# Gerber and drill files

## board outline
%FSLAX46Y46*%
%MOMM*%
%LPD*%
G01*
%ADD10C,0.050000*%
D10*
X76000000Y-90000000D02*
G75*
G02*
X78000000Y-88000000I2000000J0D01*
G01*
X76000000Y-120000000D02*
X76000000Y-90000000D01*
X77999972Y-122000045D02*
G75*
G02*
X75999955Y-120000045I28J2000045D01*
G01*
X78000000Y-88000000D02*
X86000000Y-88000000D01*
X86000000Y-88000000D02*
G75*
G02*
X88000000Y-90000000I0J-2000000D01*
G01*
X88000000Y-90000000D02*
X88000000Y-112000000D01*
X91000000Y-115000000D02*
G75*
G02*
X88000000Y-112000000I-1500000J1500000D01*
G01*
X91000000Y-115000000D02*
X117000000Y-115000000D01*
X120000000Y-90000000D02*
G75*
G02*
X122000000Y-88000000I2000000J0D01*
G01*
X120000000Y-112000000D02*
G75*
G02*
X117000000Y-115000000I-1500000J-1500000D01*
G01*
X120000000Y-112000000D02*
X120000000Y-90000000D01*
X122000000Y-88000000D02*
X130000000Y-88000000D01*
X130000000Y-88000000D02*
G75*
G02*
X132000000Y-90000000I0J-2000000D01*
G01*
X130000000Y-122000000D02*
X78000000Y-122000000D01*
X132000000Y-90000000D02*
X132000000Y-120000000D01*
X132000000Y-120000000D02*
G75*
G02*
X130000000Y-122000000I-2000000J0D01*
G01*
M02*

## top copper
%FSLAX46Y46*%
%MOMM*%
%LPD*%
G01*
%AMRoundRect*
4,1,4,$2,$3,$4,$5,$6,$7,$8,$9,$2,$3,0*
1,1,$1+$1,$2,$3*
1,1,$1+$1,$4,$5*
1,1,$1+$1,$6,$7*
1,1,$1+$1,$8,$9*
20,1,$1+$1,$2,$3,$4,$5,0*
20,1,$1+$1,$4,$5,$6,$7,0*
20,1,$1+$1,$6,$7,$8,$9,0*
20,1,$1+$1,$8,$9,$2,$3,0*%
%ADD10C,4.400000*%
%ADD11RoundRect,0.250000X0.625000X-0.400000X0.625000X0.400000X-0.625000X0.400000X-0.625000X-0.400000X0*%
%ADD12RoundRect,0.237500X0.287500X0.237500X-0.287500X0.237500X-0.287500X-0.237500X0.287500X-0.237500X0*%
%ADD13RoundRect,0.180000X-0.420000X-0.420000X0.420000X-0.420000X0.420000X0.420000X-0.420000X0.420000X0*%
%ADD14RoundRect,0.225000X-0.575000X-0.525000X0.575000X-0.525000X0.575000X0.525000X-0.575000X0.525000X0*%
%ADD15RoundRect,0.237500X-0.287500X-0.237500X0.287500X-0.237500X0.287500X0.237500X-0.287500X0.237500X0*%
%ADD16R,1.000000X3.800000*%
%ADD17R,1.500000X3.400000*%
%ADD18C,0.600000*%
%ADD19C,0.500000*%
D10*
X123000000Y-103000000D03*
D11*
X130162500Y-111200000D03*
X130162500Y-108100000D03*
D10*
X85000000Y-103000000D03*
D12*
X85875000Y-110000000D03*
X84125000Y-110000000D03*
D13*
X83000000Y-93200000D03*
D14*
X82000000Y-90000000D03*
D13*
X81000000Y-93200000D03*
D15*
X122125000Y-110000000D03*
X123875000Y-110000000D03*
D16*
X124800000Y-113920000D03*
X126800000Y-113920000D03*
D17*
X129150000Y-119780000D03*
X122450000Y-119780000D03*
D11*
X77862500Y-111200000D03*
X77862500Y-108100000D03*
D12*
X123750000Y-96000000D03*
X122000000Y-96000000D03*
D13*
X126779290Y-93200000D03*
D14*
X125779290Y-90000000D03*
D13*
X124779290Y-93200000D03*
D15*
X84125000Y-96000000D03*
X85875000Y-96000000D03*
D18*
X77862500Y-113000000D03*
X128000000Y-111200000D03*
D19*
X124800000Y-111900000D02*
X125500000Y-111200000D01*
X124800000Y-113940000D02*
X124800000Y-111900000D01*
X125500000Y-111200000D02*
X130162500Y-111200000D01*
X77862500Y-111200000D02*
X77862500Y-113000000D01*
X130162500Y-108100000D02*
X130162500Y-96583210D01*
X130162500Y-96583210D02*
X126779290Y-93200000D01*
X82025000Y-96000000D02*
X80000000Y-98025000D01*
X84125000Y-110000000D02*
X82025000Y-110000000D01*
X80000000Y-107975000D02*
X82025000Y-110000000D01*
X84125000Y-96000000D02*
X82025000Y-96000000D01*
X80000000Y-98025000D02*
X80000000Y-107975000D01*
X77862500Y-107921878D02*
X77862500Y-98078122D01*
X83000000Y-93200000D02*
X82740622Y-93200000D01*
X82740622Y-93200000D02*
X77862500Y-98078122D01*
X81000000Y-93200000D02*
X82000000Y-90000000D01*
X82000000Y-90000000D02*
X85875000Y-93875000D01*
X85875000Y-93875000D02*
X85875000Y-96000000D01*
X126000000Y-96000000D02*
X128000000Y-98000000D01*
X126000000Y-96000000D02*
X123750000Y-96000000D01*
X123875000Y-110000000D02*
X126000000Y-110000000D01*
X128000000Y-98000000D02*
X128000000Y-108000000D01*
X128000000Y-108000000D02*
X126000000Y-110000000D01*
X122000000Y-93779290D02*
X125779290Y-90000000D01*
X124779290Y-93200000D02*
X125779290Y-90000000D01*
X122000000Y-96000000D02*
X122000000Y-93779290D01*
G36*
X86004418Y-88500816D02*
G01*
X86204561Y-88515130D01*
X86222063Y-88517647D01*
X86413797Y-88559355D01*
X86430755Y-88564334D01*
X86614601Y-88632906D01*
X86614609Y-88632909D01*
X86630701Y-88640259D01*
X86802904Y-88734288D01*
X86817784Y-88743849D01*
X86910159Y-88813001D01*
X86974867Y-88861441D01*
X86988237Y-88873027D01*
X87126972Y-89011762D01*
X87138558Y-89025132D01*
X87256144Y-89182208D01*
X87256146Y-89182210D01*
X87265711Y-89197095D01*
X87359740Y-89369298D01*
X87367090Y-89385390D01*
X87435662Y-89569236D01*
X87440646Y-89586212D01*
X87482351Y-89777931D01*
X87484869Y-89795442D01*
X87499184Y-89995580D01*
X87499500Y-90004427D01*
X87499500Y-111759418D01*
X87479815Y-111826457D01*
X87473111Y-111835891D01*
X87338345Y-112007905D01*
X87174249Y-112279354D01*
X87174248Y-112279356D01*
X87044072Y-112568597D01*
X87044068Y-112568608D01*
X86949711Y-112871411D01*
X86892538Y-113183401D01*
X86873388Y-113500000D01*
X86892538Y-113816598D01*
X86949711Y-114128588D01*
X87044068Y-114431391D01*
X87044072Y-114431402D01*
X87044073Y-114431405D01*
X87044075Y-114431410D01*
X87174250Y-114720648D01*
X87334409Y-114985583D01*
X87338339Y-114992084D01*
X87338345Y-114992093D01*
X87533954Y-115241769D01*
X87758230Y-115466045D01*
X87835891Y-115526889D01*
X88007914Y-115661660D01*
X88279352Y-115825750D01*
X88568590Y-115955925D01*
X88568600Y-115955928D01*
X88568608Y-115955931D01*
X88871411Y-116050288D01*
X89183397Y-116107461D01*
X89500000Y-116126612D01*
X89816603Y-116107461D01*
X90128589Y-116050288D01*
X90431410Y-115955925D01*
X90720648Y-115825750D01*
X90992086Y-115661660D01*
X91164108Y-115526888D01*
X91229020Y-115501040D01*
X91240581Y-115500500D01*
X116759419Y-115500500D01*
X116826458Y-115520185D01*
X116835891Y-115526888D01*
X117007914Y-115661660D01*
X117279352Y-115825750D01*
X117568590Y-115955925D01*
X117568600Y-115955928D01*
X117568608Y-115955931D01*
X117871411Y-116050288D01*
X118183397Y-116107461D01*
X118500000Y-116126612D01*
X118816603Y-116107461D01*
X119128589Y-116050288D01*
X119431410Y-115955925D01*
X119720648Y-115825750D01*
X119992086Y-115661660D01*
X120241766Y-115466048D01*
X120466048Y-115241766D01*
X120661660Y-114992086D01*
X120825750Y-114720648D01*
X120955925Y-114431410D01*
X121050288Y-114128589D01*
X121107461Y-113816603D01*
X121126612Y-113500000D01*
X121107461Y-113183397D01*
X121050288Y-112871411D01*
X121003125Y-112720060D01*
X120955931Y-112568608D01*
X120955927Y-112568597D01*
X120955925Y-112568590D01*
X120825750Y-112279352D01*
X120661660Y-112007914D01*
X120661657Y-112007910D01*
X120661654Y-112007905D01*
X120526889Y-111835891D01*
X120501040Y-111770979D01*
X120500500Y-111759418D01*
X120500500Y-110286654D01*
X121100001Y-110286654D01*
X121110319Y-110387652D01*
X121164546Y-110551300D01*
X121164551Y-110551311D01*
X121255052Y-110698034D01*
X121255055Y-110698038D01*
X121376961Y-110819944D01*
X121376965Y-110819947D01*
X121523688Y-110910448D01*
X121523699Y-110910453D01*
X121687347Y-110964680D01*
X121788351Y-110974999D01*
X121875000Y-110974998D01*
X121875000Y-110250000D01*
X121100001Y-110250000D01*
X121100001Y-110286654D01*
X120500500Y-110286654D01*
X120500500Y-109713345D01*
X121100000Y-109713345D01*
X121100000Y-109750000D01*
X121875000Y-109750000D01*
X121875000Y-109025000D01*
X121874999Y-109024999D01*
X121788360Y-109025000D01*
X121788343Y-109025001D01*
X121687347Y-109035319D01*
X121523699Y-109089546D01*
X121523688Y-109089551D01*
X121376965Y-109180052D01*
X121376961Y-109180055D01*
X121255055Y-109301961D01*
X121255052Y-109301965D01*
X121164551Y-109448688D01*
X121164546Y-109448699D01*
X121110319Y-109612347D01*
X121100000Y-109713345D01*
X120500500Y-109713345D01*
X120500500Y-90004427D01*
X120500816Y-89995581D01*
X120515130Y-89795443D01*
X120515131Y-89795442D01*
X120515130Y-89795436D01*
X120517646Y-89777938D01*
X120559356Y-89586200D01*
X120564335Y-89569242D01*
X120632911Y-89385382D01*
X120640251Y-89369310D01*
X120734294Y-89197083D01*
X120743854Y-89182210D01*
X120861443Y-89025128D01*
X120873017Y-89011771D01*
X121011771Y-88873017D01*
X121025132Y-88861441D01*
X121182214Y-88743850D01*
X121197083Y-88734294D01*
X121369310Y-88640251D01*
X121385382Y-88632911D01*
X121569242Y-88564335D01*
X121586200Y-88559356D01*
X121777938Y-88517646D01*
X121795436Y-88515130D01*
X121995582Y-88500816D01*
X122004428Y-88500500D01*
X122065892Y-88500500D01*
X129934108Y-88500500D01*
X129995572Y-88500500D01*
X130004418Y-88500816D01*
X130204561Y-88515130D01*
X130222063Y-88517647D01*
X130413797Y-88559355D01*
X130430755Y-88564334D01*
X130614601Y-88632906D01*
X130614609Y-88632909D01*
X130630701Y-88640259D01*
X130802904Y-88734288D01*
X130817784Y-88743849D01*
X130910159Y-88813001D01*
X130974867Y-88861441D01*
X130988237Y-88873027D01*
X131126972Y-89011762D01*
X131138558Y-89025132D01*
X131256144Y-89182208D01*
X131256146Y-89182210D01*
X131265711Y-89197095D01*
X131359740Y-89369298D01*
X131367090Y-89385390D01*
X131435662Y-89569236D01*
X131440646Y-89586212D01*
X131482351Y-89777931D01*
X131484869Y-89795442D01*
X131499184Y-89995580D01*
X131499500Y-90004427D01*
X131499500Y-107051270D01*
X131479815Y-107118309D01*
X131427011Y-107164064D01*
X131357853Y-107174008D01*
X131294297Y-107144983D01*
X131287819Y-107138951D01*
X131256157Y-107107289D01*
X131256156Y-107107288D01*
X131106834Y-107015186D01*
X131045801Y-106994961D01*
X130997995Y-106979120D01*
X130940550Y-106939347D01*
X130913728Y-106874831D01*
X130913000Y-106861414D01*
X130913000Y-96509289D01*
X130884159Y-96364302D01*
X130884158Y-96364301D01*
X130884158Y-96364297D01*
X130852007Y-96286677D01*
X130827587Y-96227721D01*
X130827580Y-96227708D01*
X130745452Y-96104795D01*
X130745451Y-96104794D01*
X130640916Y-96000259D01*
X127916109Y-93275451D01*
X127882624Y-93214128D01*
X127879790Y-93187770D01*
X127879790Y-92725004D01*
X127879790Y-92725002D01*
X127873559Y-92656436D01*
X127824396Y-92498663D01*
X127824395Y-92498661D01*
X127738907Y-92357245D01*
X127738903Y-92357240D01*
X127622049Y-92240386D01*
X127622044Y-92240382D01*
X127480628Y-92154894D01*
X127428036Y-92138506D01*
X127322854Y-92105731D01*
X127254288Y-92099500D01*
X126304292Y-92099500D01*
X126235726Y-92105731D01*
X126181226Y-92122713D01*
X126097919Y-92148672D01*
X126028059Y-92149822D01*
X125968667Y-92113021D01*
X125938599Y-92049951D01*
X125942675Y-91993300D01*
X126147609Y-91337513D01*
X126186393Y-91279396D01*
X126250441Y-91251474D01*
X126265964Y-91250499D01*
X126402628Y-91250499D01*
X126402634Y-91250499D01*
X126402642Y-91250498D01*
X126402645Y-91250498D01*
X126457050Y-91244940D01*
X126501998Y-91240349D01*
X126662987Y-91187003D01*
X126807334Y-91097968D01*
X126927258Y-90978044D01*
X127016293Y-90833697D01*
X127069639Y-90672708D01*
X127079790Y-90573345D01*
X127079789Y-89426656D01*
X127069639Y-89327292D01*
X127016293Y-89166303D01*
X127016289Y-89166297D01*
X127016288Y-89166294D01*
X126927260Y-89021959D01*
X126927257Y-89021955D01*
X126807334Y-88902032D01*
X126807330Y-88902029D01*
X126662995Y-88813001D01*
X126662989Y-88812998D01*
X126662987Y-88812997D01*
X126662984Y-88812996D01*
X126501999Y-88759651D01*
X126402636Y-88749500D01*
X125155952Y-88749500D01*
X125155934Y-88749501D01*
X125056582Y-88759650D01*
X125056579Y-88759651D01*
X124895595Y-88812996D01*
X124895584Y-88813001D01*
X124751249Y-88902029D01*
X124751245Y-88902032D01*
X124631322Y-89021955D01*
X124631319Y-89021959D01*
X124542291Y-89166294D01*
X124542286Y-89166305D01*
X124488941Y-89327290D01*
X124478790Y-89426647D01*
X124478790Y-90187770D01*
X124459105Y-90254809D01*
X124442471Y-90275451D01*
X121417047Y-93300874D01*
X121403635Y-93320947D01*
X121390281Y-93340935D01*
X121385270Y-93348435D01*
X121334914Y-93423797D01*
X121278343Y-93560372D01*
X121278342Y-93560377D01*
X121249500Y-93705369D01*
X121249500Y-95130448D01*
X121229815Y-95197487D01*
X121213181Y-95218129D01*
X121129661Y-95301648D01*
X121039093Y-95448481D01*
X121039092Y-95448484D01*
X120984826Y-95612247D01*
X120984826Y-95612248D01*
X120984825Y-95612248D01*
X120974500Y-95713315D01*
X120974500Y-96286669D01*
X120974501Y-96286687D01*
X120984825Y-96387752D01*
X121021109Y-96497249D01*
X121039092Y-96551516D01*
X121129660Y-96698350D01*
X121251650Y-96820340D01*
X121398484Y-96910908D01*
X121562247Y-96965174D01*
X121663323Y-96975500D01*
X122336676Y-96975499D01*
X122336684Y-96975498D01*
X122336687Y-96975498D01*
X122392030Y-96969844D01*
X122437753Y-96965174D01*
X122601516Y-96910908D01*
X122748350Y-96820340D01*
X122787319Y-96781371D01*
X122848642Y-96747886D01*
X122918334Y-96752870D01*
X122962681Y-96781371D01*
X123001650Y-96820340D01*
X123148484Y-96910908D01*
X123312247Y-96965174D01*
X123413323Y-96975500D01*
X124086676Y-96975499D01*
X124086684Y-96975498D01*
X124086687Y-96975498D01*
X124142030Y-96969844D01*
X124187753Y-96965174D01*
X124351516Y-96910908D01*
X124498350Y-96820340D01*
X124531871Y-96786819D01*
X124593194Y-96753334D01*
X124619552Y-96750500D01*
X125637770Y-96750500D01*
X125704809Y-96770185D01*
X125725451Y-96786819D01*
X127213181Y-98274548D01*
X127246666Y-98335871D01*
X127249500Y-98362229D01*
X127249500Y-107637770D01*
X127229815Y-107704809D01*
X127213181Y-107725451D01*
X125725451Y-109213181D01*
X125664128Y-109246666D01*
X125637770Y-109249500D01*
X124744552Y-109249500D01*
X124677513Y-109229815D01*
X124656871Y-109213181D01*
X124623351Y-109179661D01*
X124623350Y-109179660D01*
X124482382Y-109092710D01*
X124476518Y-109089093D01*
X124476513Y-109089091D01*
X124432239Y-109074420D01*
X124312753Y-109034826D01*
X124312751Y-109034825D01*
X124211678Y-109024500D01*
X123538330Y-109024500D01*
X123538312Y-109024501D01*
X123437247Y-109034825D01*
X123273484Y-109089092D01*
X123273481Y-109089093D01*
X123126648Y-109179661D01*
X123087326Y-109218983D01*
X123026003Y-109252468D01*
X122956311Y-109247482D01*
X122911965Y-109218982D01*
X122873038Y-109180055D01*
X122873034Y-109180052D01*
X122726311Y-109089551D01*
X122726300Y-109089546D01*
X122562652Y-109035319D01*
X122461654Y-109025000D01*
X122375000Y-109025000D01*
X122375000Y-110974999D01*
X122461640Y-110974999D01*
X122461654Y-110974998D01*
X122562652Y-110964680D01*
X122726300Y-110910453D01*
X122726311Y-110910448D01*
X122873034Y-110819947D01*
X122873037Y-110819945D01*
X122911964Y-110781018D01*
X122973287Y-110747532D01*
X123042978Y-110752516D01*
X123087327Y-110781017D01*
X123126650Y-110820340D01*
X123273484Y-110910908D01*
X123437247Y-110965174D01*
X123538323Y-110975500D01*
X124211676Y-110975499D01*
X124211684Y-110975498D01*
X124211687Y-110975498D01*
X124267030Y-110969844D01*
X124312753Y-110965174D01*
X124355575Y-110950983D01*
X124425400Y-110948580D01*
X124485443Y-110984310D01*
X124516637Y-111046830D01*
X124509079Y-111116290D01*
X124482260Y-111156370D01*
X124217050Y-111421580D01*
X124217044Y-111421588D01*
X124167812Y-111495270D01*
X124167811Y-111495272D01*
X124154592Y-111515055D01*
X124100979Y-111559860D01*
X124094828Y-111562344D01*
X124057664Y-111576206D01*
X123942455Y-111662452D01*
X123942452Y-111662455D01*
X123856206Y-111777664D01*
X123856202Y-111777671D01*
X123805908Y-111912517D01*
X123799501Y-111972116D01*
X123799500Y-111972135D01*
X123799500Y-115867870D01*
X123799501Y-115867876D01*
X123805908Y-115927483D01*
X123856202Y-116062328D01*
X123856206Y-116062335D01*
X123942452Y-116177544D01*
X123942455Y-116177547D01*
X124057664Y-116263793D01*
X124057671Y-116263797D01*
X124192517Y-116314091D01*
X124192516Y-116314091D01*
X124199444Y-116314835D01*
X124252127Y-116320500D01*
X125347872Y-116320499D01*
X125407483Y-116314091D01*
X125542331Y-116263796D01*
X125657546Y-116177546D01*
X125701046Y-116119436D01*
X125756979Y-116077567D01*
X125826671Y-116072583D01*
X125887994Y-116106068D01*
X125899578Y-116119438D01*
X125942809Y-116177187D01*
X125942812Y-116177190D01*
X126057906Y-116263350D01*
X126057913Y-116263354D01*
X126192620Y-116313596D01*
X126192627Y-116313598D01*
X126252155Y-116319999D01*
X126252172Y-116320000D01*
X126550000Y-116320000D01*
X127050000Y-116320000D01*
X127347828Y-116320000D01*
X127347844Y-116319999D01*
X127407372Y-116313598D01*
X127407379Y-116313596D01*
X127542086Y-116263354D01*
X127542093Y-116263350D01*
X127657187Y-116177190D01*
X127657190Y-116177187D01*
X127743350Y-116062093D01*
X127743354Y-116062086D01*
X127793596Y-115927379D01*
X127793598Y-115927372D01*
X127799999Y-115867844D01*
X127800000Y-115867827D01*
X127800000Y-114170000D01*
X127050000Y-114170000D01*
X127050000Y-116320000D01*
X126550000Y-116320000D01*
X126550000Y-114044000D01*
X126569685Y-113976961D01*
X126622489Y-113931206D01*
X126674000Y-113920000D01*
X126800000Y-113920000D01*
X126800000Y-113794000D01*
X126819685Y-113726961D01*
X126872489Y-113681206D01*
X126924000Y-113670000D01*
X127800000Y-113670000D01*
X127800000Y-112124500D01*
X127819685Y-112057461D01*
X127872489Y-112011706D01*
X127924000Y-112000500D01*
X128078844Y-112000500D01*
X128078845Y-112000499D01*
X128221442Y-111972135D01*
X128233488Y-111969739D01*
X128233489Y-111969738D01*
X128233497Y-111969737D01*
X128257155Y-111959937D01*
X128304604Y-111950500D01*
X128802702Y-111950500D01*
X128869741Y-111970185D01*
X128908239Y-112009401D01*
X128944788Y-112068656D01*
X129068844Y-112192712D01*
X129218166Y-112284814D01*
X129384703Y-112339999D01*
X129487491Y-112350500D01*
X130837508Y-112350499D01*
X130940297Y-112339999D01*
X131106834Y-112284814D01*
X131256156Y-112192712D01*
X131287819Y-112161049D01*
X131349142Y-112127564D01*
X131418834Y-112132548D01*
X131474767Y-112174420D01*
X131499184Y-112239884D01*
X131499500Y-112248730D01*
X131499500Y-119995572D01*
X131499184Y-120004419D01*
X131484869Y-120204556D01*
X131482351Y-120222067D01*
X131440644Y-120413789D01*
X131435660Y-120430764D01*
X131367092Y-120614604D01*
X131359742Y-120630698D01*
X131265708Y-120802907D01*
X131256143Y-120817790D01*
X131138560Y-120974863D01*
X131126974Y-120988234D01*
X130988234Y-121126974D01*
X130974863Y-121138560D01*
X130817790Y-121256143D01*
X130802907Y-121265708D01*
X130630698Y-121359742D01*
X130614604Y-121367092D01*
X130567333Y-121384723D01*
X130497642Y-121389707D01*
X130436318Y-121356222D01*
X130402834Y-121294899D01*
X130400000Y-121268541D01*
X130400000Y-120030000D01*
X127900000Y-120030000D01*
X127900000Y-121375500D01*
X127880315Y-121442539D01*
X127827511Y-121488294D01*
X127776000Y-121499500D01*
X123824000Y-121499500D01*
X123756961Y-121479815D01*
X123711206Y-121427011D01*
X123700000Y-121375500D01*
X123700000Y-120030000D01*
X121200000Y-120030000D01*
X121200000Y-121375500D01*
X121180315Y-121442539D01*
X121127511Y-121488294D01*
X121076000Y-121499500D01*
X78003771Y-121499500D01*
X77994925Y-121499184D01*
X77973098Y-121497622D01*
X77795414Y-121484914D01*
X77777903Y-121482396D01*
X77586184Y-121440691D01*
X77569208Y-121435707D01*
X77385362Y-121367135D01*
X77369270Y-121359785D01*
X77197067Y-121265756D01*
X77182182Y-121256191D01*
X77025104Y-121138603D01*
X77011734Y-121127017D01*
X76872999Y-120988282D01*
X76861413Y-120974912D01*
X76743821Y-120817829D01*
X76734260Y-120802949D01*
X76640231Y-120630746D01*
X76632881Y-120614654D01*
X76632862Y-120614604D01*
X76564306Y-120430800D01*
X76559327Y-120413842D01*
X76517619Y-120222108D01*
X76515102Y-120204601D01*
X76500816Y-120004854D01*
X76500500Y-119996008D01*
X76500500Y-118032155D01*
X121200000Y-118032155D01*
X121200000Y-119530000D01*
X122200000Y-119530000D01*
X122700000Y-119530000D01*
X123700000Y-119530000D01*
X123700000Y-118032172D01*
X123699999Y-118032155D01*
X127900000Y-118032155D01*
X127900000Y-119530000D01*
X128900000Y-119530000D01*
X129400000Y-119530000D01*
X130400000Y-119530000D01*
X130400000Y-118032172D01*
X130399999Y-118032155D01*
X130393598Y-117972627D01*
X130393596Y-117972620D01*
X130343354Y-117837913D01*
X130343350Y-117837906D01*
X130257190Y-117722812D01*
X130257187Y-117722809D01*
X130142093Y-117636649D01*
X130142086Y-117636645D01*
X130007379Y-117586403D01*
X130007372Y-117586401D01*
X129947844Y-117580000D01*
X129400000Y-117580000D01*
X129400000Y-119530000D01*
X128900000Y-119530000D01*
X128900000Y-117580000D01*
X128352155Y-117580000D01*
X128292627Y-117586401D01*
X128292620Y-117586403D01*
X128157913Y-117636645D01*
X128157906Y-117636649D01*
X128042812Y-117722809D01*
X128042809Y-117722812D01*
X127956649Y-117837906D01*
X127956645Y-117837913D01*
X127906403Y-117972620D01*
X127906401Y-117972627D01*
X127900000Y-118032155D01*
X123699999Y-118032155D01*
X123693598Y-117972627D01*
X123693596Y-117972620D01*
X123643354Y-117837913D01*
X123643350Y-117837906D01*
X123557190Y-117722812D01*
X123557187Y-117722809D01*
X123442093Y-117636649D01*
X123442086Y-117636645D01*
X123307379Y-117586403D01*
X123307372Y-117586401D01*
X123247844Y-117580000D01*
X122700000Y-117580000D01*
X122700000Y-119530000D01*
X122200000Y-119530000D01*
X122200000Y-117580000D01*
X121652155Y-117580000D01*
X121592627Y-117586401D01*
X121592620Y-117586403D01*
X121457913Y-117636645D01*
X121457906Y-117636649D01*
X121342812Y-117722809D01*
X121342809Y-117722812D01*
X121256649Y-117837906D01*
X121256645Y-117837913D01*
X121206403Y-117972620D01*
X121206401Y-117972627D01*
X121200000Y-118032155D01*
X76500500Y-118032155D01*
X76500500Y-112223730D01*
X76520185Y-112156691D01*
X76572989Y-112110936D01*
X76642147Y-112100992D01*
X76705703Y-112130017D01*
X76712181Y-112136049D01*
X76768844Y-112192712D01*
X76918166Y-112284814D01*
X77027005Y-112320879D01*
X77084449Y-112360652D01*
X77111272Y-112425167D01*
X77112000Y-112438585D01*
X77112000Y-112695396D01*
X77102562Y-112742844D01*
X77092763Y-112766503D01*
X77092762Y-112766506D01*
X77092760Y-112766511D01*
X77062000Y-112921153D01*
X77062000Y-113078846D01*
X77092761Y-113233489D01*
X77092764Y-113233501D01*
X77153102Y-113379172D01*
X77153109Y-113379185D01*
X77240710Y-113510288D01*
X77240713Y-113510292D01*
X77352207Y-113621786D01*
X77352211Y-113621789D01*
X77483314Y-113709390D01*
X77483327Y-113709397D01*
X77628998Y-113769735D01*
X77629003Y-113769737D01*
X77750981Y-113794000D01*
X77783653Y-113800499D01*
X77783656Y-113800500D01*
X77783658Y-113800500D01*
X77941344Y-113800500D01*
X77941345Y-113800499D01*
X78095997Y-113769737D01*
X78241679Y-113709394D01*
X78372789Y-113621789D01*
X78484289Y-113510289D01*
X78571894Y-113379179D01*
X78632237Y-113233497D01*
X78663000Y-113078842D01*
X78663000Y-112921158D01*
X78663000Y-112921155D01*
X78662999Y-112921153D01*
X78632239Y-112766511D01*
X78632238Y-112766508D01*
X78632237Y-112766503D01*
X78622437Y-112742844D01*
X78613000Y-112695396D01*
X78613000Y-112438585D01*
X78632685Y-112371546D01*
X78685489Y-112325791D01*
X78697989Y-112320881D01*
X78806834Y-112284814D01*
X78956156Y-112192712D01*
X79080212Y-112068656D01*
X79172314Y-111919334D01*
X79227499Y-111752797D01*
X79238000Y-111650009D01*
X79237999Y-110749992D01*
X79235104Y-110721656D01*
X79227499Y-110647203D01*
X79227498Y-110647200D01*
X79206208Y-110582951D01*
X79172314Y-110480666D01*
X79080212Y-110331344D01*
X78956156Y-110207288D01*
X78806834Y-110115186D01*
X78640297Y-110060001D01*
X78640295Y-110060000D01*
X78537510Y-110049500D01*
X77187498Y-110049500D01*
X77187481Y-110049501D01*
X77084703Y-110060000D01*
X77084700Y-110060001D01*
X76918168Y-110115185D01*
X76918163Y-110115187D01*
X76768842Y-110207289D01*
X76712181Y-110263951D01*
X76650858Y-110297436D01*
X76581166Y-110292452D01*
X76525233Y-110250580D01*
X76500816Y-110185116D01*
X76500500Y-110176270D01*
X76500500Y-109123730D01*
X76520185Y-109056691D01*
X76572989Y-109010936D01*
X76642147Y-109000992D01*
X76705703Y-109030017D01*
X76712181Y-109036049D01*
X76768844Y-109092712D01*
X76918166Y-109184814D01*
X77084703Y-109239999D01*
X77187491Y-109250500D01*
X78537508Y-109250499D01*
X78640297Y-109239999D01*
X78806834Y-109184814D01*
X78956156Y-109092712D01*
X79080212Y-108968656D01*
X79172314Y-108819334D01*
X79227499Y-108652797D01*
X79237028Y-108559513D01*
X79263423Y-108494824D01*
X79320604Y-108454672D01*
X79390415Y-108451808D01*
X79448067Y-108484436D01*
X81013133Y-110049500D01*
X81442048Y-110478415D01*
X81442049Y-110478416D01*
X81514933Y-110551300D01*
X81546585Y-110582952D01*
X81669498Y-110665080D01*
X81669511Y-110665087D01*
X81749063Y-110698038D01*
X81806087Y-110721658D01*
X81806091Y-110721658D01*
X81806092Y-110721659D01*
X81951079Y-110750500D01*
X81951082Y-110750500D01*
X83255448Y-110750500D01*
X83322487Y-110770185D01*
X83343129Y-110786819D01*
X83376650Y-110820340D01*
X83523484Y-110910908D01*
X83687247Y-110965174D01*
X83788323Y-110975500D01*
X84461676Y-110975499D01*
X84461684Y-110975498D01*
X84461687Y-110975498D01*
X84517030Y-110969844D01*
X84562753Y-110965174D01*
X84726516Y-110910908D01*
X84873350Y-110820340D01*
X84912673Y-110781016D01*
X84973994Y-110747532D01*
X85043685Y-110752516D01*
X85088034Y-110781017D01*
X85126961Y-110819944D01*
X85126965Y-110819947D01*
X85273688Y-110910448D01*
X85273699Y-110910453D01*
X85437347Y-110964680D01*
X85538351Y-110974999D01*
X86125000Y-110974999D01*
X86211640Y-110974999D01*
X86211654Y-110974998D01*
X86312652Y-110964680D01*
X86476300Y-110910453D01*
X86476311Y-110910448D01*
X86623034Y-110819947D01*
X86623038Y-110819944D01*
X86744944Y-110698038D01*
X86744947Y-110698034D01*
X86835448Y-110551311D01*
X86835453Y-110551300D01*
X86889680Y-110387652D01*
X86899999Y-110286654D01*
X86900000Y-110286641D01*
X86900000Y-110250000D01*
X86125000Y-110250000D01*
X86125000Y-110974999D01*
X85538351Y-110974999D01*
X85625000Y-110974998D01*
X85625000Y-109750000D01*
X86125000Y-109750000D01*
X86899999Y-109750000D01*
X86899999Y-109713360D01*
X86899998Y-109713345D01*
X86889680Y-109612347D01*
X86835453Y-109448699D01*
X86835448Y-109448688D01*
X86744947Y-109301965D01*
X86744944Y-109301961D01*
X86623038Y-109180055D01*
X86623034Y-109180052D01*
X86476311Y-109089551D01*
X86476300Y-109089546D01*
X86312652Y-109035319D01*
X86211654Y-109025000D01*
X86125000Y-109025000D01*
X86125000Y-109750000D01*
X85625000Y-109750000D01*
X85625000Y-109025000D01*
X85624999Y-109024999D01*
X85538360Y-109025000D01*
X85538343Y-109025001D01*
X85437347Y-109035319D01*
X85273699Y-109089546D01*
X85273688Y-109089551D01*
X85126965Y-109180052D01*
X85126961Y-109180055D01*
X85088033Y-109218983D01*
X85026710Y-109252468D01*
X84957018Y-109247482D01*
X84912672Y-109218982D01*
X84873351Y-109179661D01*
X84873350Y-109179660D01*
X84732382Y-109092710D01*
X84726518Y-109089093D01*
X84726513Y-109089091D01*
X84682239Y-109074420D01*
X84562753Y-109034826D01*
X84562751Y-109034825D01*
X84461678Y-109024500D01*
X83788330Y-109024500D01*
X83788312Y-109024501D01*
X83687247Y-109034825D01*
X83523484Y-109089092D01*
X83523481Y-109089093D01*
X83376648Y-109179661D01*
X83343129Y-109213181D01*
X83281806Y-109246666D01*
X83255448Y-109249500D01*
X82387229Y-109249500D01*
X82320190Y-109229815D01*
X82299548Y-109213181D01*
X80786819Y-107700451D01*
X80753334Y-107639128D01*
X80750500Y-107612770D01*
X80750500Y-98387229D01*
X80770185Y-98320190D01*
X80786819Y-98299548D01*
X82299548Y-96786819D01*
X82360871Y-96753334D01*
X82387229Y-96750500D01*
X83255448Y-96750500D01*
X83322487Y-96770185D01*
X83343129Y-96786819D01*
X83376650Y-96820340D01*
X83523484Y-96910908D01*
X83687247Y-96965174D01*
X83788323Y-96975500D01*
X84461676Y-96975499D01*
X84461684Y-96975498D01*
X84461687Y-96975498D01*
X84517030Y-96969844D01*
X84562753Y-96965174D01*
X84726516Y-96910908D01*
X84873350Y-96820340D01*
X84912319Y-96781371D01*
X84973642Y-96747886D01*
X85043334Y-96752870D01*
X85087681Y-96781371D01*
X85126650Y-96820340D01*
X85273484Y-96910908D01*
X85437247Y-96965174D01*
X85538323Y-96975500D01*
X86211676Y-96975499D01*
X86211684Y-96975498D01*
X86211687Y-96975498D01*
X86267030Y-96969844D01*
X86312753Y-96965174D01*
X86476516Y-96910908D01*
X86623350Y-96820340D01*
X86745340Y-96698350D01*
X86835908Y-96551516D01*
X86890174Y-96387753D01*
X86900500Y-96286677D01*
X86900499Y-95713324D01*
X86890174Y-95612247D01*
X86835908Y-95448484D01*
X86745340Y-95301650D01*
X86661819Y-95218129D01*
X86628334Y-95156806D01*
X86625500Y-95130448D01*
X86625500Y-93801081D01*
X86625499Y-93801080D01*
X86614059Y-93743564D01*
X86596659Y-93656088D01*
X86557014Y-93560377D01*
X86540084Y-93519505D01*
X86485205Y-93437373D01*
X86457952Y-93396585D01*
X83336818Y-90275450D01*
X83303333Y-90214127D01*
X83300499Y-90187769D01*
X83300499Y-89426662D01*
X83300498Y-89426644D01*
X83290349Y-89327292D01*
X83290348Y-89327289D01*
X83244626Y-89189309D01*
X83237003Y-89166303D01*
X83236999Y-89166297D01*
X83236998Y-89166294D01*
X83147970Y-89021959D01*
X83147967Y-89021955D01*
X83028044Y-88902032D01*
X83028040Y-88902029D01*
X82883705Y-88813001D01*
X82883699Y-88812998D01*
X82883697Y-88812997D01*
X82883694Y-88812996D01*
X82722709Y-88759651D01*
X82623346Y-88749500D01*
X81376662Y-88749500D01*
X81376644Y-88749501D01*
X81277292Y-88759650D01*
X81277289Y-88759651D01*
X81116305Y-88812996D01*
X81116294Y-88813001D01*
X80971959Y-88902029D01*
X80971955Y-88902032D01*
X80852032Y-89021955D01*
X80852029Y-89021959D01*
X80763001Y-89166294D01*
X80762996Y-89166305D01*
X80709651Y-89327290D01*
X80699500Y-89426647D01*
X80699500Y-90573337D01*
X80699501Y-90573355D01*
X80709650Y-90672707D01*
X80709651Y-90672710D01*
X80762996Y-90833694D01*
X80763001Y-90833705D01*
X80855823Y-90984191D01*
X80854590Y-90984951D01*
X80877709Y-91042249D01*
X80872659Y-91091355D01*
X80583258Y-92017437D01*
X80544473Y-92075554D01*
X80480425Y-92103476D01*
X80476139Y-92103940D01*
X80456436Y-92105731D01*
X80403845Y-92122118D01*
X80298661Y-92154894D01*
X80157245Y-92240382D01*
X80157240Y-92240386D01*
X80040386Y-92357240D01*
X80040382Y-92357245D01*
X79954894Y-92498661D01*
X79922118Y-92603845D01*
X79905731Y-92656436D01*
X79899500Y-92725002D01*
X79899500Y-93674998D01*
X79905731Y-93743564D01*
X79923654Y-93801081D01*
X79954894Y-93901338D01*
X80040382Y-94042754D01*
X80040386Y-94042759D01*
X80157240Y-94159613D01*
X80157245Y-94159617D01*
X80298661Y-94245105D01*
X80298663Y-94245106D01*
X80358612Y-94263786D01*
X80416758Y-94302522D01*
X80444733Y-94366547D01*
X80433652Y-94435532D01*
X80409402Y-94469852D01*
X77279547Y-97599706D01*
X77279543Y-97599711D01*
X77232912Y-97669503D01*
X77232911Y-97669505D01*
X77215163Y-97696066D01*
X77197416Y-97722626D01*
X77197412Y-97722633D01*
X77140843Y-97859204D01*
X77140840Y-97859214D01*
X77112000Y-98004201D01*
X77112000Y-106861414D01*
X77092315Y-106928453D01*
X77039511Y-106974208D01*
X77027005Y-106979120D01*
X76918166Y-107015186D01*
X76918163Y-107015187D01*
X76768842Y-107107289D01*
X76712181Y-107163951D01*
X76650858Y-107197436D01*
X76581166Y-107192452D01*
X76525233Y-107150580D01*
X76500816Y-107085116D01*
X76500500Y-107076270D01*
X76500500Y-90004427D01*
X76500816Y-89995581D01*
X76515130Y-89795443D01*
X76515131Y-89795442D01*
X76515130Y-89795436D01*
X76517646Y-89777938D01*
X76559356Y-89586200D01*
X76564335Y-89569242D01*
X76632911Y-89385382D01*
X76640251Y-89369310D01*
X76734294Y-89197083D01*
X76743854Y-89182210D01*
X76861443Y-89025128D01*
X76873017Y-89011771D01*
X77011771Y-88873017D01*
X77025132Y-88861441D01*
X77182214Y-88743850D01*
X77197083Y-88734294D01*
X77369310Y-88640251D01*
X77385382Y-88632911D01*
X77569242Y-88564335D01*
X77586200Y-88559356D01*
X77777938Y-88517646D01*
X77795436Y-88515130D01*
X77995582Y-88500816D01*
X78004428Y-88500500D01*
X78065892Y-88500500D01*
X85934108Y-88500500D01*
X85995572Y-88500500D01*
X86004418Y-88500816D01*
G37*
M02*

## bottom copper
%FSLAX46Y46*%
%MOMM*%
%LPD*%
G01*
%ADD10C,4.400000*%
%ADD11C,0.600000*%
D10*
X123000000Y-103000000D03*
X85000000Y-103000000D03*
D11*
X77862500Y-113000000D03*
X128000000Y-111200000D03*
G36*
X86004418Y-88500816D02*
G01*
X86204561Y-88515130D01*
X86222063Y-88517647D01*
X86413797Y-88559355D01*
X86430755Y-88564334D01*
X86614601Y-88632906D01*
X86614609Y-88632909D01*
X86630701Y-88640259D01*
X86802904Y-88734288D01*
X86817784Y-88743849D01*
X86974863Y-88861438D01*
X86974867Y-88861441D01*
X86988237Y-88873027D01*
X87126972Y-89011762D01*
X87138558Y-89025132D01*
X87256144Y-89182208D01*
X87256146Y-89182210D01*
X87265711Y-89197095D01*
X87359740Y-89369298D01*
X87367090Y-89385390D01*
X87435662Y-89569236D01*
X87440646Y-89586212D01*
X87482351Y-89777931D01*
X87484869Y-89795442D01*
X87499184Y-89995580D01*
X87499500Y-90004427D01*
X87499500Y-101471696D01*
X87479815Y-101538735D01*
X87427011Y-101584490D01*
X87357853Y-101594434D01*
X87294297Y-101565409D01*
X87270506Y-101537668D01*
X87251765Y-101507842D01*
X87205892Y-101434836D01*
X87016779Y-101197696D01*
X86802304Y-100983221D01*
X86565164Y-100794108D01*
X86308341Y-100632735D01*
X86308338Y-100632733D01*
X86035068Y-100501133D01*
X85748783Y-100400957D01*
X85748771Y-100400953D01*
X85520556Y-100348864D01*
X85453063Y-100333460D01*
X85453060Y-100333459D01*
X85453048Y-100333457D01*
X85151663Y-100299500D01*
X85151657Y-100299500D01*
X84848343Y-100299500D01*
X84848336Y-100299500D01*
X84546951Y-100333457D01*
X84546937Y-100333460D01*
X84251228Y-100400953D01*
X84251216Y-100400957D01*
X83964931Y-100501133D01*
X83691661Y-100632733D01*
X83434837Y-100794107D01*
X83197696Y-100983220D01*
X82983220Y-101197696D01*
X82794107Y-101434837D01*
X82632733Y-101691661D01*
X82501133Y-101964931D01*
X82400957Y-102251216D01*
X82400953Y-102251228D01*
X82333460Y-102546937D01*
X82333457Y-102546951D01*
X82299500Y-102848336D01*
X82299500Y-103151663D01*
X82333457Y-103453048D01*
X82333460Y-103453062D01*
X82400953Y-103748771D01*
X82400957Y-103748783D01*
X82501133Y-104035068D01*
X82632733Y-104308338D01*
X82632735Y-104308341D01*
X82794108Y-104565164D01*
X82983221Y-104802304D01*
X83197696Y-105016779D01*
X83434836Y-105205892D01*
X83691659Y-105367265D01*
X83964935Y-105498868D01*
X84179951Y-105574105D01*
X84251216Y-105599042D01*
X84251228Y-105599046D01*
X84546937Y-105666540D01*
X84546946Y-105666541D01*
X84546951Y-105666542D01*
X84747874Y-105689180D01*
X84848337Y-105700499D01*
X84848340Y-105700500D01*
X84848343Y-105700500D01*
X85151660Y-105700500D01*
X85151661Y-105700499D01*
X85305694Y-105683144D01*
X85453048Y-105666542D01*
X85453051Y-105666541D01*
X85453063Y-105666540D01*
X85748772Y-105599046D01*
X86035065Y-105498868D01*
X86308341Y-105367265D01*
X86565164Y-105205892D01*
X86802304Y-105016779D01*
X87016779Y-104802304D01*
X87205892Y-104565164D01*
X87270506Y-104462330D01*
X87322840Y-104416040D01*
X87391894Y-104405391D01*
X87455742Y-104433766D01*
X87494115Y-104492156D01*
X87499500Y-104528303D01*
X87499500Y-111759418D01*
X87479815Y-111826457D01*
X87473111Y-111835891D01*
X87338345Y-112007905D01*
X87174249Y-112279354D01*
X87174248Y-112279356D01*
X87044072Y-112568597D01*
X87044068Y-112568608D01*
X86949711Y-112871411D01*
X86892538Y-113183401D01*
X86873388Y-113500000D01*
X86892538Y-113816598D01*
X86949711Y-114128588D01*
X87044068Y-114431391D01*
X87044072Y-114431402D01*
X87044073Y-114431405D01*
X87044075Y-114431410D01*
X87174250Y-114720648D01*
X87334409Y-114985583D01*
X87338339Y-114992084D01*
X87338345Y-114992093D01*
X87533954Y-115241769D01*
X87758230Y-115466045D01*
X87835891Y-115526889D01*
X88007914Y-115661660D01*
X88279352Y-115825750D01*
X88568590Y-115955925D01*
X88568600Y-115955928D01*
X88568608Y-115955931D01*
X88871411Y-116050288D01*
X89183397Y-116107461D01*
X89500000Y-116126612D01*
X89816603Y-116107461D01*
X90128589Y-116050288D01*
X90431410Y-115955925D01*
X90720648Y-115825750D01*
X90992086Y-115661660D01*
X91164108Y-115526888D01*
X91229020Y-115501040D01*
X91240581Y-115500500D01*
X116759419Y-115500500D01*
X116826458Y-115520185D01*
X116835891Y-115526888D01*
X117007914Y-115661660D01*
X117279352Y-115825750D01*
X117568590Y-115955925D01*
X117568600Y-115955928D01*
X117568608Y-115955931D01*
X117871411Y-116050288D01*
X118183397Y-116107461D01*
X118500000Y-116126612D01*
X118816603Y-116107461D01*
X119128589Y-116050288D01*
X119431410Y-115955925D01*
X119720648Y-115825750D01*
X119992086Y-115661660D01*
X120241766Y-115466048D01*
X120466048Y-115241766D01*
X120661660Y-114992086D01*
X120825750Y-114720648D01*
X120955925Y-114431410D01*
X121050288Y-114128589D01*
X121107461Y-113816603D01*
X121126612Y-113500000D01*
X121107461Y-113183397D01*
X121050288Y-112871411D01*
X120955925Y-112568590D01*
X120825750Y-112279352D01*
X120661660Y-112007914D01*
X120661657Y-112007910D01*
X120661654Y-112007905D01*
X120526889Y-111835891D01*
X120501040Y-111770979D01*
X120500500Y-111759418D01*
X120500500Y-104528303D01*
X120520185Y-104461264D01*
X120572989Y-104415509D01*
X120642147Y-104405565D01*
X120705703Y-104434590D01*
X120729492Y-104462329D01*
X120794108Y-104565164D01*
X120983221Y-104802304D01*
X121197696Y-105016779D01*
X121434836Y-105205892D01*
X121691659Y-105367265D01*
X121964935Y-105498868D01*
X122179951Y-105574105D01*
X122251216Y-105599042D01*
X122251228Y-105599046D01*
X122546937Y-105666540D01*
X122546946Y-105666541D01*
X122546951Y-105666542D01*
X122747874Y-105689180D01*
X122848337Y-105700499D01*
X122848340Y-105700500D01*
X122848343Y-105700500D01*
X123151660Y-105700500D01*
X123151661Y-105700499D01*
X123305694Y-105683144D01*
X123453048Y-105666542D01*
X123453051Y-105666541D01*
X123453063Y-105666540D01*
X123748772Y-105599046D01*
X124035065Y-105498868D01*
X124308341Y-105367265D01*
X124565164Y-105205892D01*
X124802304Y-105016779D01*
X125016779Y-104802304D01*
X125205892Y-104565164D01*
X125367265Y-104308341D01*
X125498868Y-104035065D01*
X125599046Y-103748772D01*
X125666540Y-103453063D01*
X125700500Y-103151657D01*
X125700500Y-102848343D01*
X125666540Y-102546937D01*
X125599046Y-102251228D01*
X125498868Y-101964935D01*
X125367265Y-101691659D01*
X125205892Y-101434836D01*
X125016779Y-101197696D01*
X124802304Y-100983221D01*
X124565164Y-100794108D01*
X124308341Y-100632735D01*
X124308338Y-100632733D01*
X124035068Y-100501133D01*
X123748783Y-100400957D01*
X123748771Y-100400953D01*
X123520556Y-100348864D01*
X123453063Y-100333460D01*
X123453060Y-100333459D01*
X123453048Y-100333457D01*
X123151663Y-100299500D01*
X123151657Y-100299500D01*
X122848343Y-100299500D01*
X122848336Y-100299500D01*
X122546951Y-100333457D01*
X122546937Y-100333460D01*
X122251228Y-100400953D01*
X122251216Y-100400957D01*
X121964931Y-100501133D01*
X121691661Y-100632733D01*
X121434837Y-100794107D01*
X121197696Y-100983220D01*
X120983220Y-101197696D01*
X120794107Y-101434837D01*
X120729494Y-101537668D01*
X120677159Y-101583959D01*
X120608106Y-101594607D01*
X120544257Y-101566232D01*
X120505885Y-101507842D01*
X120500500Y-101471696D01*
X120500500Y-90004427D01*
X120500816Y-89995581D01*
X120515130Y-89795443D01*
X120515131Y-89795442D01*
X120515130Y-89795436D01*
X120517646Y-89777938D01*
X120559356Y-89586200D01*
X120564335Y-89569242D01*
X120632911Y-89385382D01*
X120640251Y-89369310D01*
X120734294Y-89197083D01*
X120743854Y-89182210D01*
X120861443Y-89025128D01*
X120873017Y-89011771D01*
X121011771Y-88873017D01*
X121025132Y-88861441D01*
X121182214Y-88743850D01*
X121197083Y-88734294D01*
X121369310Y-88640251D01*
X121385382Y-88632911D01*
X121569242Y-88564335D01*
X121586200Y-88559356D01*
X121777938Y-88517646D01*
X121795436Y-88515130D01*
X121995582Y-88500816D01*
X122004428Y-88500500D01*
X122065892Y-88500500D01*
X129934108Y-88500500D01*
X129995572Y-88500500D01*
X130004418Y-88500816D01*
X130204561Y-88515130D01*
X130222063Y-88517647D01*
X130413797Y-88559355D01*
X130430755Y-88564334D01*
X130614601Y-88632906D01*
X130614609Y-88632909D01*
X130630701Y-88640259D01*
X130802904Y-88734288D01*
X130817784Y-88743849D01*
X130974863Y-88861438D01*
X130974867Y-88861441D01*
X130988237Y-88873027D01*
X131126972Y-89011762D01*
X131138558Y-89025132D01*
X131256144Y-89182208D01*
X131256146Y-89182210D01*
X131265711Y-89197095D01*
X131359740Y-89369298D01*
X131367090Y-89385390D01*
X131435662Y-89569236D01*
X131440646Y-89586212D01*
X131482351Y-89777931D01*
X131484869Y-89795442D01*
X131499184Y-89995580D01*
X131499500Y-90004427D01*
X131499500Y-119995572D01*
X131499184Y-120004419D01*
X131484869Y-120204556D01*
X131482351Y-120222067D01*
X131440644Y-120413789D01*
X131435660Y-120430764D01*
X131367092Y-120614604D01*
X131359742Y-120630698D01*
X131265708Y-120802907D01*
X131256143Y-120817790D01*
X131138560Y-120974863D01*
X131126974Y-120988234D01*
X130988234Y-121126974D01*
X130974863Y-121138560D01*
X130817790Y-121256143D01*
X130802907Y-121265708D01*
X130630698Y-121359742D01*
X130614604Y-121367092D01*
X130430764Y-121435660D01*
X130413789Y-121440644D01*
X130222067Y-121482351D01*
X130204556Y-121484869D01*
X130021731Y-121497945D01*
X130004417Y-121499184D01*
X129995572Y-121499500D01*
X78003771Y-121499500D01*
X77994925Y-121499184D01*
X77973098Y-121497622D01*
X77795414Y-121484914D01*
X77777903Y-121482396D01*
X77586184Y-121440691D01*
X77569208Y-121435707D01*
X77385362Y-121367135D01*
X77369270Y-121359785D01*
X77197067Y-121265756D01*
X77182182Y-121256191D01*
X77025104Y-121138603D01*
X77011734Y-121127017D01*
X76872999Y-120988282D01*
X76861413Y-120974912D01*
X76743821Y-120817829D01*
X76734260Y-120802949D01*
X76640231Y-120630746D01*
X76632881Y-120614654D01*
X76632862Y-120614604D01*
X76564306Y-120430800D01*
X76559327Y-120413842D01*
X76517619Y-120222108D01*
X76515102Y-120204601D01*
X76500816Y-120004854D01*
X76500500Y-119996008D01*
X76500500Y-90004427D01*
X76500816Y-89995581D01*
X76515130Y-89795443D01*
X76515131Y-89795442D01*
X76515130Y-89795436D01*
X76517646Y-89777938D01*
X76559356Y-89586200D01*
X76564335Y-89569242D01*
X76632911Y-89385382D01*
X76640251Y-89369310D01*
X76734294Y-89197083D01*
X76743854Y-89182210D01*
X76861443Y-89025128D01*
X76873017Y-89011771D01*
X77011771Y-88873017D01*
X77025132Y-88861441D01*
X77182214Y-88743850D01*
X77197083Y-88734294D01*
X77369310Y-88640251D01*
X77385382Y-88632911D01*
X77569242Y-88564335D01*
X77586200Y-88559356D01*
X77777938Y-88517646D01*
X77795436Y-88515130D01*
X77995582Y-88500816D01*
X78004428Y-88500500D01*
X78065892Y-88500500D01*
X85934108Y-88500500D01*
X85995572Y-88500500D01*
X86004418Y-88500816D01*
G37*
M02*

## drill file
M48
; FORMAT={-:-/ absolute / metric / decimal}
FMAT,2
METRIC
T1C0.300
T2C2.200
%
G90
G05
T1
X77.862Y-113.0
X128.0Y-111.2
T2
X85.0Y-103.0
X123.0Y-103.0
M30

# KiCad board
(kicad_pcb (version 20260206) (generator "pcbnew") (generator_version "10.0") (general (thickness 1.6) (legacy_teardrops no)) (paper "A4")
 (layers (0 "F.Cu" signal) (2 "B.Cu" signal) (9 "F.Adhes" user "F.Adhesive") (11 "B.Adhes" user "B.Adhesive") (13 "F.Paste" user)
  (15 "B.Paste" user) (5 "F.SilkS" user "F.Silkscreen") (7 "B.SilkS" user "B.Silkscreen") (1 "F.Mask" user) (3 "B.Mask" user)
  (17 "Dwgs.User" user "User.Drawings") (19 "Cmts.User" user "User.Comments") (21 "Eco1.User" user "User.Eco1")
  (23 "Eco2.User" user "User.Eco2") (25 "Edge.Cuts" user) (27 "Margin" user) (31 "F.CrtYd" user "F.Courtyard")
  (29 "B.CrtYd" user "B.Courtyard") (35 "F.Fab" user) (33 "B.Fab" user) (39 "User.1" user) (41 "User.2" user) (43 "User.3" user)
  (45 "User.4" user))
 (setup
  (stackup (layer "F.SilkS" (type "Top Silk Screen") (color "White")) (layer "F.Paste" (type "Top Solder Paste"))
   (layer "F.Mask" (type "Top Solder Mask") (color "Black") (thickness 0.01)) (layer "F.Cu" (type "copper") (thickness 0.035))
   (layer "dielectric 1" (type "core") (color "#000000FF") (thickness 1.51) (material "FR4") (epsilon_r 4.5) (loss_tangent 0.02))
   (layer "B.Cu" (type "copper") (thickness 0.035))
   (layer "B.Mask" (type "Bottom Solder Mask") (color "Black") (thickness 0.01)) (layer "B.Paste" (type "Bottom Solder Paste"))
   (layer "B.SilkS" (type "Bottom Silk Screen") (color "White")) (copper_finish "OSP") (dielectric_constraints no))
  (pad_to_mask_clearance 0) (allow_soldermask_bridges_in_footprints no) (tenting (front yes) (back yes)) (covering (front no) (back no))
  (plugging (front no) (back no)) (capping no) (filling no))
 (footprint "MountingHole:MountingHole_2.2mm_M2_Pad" (layer "F.Cu") (at 123 103)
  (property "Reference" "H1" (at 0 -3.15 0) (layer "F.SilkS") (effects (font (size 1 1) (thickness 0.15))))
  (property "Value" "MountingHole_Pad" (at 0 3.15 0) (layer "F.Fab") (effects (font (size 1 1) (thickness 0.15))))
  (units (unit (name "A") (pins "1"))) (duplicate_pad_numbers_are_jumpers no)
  (pad "1" thru_hole circle (at 0 0) (size 4.4 4.4) (drill 2.2) (layers "*.Cu" "*.Mask") (remove_unused_layers no) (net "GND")
   (zone_connect 2)))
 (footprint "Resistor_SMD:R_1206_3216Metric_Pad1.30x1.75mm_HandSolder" (layer "F.Cu") (at 130.1625 109.65 90)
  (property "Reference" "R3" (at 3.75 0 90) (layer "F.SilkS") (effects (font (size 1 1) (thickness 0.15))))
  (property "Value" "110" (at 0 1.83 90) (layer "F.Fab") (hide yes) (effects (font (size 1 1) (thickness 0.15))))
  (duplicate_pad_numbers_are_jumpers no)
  (pad "1" smd roundrect (at -1.55 0 90) (size 1.3 1.75) (layers "F.Cu" "F.Mask" "F.Paste") (roundrect_rratio 0.192308) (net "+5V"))
  (pad "2" smd roundrect (at 1.55 0 90) (size 1.3 1.75) (layers "F.Cu" "F.Mask" "F.Paste") (roundrect_rratio 0.192308) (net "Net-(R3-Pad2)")))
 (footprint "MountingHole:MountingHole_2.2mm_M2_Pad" (layer "F.Cu") (at 85 103)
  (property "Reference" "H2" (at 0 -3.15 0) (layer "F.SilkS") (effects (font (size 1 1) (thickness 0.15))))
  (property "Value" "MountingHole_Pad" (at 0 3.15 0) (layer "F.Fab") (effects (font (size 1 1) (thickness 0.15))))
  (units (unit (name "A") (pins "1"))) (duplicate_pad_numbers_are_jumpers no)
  (pad "1" thru_hole circle (at 0 0) (size 4.4 4.4) (drill 2.2) (layers "*.Cu" "*.Mask") (remove_unused_layers no) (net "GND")
   (zone_connect 2)))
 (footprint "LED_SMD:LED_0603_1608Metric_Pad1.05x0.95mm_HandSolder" (layer "F.Cu") (at 85 110 180)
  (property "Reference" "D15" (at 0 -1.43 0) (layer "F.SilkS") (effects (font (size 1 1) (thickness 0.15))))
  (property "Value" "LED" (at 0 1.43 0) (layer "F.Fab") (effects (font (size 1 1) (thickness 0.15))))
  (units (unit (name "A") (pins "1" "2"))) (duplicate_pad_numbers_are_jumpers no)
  (pad "1" smd roundrect (at -0.875 0 180) (size 1.05 0.95) (layers "F.Cu" "F.Mask" "F.Paste") (roundrect_rratio 0.25) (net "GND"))
  (pad "2" smd roundrect (at 0.875 0 180) (size 1.05 0.95) (layers "F.Cu" "F.Mask" "F.Paste") (roundrect_rratio 0.25) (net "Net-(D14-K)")))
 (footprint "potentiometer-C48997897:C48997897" (layer "F.Cu") (at 82 95.4)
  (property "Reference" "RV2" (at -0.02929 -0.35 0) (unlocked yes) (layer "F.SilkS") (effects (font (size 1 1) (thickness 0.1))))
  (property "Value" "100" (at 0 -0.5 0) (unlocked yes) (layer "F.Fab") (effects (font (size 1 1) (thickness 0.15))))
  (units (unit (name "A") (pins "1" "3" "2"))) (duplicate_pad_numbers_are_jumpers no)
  (pad "1" smd roundrect (at 1 -2.2) (size 1.2 1.2) (layers "F.Cu" "F.Mask" "F.Paste") (roundrect_rratio 0.15) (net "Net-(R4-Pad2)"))
  (pad "2" smd roundrect (at 0 -5.4) (size 1.6 1.5) (layers "F.Cu" "F.Mask" "F.Paste") (roundrect_rratio 0.15) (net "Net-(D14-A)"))
  (pad "3" smd roundrect (at -1 -2.2) (size 1.2 1.2) (layers "F.Cu" "F.Mask" "F.Paste") (roundrect_rratio 0.15) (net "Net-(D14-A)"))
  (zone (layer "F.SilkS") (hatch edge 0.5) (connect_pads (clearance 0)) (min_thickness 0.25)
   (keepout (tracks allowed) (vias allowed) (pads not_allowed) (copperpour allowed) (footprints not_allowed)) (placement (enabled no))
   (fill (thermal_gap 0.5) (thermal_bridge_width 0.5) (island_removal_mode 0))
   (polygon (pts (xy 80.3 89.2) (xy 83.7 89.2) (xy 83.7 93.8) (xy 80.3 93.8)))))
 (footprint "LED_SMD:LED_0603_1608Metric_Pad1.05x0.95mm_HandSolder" (layer "F.Cu") (at 123 110)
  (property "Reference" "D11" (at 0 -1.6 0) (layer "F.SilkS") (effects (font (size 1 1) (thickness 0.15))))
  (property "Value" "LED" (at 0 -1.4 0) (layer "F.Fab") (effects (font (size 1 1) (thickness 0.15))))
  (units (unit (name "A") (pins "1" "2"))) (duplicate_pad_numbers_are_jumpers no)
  (pad "1" smd roundrect (at -0.875 0) (size 1.05 0.95) (layers "F.Cu" "F.Mask" "F.Paste") (roundrect_rratio 0.25) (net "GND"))
  (pad "2" smd roundrect (at 0.875 0) (size 1.05 0.95) (layers "F.Cu" "F.Mask" "F.Paste") (roundrect_rratio 0.25) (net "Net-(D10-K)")))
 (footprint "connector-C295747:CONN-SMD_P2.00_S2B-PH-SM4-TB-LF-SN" (layer "F.Cu") (at 125.8 116.85)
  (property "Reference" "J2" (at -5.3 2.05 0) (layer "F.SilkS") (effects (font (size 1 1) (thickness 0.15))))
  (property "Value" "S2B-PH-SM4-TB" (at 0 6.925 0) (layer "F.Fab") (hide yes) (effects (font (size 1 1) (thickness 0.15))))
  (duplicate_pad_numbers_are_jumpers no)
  (pad "1" smd rect (at -1 -2.93) (size 1 3.8) (layers "F.Cu" "F.Mask" "F.Paste") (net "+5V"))
  (pad "2" smd rect (at 1 -2.93) (size 1 3.8) (layers "F.Cu" "F.Mask" "F.Paste") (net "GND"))
  (pad "3" smd rect (at 3.35 2.93) (size 1.5 3.4) (layers "F.Cu" "F.Mask" "F.Paste") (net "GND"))
  (pad "4" smd rect (at -3.35 2.93) (size 1.5 3.4) (layers "F.Cu" "F.Mask" "F.Paste") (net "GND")))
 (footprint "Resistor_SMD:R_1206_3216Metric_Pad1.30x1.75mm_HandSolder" (layer "F.Cu") (at 77.8625 109.65 90)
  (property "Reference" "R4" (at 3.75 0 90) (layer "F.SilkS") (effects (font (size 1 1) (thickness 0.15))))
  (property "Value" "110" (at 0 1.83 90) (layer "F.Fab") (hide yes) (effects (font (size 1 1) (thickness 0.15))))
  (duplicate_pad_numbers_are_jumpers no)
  (pad "1" smd roundrect (at -1.55 0 90) (size 1.3 1.75) (layers "F.Cu" "F.Mask" "F.Paste") (roundrect_rratio 0.192308) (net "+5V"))
  (pad "2" smd roundrect (at 1.55 0 90) (size 1.3 1.75) (layers "F.Cu" "F.Mask" "F.Paste") (roundrect_rratio 0.192308) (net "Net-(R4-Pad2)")))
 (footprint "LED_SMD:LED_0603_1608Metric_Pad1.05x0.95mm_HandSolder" (layer "F.Cu") (at 122.875 96 180)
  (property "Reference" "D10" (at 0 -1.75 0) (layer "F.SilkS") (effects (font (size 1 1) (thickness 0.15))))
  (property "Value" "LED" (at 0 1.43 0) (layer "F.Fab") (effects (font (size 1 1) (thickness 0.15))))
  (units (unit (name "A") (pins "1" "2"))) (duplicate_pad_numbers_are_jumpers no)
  (pad "1" smd roundrect (at -0.875 0 180) (size 1.05 0.95) (layers "F.Cu" "F.Mask" "F.Paste") (roundrect_rratio 0.25) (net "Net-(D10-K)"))
  (pad "2" smd roundrect (at 0.875 0 180) (size 1.05 0.95) (layers "F.Cu" "F.Mask" "F.Paste") (roundrect_rratio 0.25) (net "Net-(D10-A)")))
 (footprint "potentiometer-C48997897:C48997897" (layer "F.Cu") (at 125.77929 95.4)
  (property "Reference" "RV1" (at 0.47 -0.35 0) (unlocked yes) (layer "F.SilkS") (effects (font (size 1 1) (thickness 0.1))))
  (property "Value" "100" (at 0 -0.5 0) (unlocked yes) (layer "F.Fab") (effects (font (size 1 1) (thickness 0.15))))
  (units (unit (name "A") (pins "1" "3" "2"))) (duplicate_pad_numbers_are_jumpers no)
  (pad "1" smd roundrect (at 1 -2.2) (size 1.2 1.2) (layers "F.Cu" "F.Mask" "F.Paste") (roundrect_rratio 0.15) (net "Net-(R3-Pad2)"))
  (pad "2" smd roundrect (at 0 -5.4) (size 1.6 1.5) (layers "F.Cu" "F.Mask" "F.Paste") (roundrect_rratio 0.15) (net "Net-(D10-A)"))
  (pad "3" smd roundrect (at -1 -2.2) (size 1.2 1.2) (layers "F.Cu" "F.Mask" "F.Paste") (roundrect_rratio 0.15) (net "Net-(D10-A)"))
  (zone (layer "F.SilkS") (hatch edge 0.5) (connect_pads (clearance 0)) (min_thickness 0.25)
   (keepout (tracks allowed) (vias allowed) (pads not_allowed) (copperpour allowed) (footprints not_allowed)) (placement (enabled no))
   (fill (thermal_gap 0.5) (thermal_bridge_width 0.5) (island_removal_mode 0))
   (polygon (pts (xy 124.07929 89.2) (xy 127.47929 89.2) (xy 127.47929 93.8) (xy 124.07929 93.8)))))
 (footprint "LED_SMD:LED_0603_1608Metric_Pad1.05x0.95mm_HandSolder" (layer "F.Cu") (at 85 96)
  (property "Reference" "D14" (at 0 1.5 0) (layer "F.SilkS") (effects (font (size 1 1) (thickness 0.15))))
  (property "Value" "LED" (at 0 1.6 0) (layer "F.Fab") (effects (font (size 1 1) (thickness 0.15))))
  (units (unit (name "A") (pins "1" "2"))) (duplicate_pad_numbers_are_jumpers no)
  (pad "1" smd roundrect (at -0.875 0) (size 1.05 0.95) (layers "F.Cu" "F.Mask" "F.Paste") (roundrect_rratio 0.25) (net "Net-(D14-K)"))
  (pad "2" smd roundrect (at 0.875 0) (size 1.05 0.95) (layers "F.Cu" "F.Mask" "F.Paste") (roundrect_rratio 0.25) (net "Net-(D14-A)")))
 (gr_arc (start 76 90) (mid 76.585786 88.585786) (end 78 88) (stroke (width 0.05) (type default)) (layer "Edge.Cuts"))
 (gr_line (start 76 120) (end 76 90) (stroke (width 0.05) (type default)) (layer "Edge.Cuts"))
 (gr_arc (start 77.999972 122.000045) (mid 76.585758 121.414258) (end 75.999972 120.000045) (stroke (width 0.05) (type default))
  (layer "Edge.Cuts"))
 (gr_line (start 78 88) (end 86 88) (stroke (width 0.05) (type default)) (layer "Edge.Cuts"))
 (gr_arc (start 86 88) (mid 87.414213 88.585786) (end 88 90) (stroke (width 0.05) (type default)) (layer "Edge.Cuts"))
 (gr_line (start 88 90) (end 88 112) (stroke (width 0.05) (type default)) (layer "Edge.Cuts"))
 (gr_arc (start 91 115) (mid 88 115) (end 88 112) (stroke (width 0.05) (type default)) (layer "Edge.Cuts"))
 (gr_line (start 91 115) (end 117 115) (stroke (width 0.05) (type default)) (layer "Edge.Cuts"))
 (gr_arc (start 120 90) (mid 120.585786 88.585786) (end 122 88) (stroke (width 0.05) (type default)) (layer "Edge.Cuts"))
 (gr_arc (start 120 112) (mid 120 115) (end 117 115) (stroke (width 0.05) (type default)) (layer "Edge.Cuts"))
 (gr_line (start 120 112) (end 120 90) (stroke (width 0.05) (type default)) (layer "Edge.Cuts"))
 (gr_line (start 122 88) (end 130 88) (stroke (width 0.05) (type default)) (layer "Edge.Cuts"))
 (gr_arc (start 130 88) (mid 131.414213 88.585786) (end 132 90) (stroke (width 0.05) (type default)) (layer "Edge.Cuts"))
 (gr_line (start 130 122) (end 78 122) (stroke (width 0.05) (type default)) (layer "Edge.Cuts"))
 (gr_line (start 132 90) (end 132 120) (stroke (width 0.05) (type default)) (layer "Edge.Cuts"))
 (gr_arc (start 132 120) (mid 131.414213 121.414213) (end 130 122) (stroke (width 0.05) (type default)) (layer "Edge.Cuts"))
 (segment (start 124.8 111.9) (end 125.5 111.2) (width 0.5) (layer "F.Cu") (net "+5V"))
 (segment (start 124.8 113.94) (end 124.8 111.9) (width 0.5) (layer "F.Cu") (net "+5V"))
 (segment (start 125.5 111.2) (end 130.1625 111.2) (width 0.5) (layer "F.Cu") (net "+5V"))
 (segment (start 77.8625 111.2) (end 77.8625 113) (width 0.5) (layer "F.Cu") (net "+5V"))
 (via (at 77.8625 113) (size 0.6) (drill 0.3) (layers "F.Cu" "B.Cu") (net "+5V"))
 (via (at 128 111.2) (size 0.6) (drill 0.3) (layers "F.Cu" "B.Cu") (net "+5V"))
 (segment (start 130.1625 108.1) (end 130.1625 96.58321) (width 0.5) (layer "F.Cu") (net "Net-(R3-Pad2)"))
 (segment (start 130.1625 96.58321) (end 126.77929 93.2) (width 0.5) (layer "F.Cu") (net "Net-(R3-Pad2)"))
 (segment (start 82.025 96) (end 80 98.025) (width 0.5) (layer "F.Cu") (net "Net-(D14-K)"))
 (segment (start 84.125 110) (end 82.025 110) (width 0.5) (layer "F.Cu") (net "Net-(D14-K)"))
 (segment (start 80 107.975) (end 82.025 110) (width 0.5) (layer "F.Cu") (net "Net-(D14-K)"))
 (segment (start 84.125 96) (end 82.025 96) (width 0.5) (layer "F.Cu") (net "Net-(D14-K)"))
 (segment (start 80 98.025) (end 80 107.975) (width 0.5) (layer "F.Cu") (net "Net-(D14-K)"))
 (segment (start 77.8625 107.921878) (end 77.8625 98.078122) (width 0.5) (layer "F.Cu") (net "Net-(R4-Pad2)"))
 (segment (start 83 93.2) (end 82.740622 93.2) (width 0.5) (layer "F.Cu") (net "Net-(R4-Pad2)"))
 (segment (start 82.740622 93.2) (end 77.8625 98.078122) (width 0.5) (layer "F.Cu") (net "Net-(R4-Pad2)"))
 (segment (start 81 93.2) (end 82 90) (width 0.5) (layer "F.Cu") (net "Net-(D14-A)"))
 (segment (start 82 90) (end 85.875 93.875) (width 0.5) (layer "F.Cu") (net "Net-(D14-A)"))
 (segment (start 85.875 93.875) (end 85.875 96) (width 0.5) (layer "F.Cu") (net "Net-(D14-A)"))
 (segment (start 126 96) (end 128 98) (width 0.5) (layer "F.Cu") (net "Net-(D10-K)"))
 (segment (start 126 96) (end 123.75 96) (width 0.5) (layer "F.Cu") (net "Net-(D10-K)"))
 (segment (start 123.875 110) (end 126 110) (width 0.5) (layer "F.Cu") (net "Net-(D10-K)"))
 (segment (start 128 98) (end 128 108) (width 0.5) (layer "F.Cu") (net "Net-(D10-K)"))
 (segment (start 128 108) (end 126 110) (width 0.5) (layer "F.Cu") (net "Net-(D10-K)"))
 (segment (start 122 93.77929) (end 125.77929 90) (width 0.5) (layer "F.Cu") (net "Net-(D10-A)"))
 (segment (start 124.77929 93.2) (end 125.77929 90) (width 0.5) (layer "F.Cu") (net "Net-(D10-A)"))
 (segment (start 122 96) (end 122 93.77929) (width 0.5) (layer "F.Cu") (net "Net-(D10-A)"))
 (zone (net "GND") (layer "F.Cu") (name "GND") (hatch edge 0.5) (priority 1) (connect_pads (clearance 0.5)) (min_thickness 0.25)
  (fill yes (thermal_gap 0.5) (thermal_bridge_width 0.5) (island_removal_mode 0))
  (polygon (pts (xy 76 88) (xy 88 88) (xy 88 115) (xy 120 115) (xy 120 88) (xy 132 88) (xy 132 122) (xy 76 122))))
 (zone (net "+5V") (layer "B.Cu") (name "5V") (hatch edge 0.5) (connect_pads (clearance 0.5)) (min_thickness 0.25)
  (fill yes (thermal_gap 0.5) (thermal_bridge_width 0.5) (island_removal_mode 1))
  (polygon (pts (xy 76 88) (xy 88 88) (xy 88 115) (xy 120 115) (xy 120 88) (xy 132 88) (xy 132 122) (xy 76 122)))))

